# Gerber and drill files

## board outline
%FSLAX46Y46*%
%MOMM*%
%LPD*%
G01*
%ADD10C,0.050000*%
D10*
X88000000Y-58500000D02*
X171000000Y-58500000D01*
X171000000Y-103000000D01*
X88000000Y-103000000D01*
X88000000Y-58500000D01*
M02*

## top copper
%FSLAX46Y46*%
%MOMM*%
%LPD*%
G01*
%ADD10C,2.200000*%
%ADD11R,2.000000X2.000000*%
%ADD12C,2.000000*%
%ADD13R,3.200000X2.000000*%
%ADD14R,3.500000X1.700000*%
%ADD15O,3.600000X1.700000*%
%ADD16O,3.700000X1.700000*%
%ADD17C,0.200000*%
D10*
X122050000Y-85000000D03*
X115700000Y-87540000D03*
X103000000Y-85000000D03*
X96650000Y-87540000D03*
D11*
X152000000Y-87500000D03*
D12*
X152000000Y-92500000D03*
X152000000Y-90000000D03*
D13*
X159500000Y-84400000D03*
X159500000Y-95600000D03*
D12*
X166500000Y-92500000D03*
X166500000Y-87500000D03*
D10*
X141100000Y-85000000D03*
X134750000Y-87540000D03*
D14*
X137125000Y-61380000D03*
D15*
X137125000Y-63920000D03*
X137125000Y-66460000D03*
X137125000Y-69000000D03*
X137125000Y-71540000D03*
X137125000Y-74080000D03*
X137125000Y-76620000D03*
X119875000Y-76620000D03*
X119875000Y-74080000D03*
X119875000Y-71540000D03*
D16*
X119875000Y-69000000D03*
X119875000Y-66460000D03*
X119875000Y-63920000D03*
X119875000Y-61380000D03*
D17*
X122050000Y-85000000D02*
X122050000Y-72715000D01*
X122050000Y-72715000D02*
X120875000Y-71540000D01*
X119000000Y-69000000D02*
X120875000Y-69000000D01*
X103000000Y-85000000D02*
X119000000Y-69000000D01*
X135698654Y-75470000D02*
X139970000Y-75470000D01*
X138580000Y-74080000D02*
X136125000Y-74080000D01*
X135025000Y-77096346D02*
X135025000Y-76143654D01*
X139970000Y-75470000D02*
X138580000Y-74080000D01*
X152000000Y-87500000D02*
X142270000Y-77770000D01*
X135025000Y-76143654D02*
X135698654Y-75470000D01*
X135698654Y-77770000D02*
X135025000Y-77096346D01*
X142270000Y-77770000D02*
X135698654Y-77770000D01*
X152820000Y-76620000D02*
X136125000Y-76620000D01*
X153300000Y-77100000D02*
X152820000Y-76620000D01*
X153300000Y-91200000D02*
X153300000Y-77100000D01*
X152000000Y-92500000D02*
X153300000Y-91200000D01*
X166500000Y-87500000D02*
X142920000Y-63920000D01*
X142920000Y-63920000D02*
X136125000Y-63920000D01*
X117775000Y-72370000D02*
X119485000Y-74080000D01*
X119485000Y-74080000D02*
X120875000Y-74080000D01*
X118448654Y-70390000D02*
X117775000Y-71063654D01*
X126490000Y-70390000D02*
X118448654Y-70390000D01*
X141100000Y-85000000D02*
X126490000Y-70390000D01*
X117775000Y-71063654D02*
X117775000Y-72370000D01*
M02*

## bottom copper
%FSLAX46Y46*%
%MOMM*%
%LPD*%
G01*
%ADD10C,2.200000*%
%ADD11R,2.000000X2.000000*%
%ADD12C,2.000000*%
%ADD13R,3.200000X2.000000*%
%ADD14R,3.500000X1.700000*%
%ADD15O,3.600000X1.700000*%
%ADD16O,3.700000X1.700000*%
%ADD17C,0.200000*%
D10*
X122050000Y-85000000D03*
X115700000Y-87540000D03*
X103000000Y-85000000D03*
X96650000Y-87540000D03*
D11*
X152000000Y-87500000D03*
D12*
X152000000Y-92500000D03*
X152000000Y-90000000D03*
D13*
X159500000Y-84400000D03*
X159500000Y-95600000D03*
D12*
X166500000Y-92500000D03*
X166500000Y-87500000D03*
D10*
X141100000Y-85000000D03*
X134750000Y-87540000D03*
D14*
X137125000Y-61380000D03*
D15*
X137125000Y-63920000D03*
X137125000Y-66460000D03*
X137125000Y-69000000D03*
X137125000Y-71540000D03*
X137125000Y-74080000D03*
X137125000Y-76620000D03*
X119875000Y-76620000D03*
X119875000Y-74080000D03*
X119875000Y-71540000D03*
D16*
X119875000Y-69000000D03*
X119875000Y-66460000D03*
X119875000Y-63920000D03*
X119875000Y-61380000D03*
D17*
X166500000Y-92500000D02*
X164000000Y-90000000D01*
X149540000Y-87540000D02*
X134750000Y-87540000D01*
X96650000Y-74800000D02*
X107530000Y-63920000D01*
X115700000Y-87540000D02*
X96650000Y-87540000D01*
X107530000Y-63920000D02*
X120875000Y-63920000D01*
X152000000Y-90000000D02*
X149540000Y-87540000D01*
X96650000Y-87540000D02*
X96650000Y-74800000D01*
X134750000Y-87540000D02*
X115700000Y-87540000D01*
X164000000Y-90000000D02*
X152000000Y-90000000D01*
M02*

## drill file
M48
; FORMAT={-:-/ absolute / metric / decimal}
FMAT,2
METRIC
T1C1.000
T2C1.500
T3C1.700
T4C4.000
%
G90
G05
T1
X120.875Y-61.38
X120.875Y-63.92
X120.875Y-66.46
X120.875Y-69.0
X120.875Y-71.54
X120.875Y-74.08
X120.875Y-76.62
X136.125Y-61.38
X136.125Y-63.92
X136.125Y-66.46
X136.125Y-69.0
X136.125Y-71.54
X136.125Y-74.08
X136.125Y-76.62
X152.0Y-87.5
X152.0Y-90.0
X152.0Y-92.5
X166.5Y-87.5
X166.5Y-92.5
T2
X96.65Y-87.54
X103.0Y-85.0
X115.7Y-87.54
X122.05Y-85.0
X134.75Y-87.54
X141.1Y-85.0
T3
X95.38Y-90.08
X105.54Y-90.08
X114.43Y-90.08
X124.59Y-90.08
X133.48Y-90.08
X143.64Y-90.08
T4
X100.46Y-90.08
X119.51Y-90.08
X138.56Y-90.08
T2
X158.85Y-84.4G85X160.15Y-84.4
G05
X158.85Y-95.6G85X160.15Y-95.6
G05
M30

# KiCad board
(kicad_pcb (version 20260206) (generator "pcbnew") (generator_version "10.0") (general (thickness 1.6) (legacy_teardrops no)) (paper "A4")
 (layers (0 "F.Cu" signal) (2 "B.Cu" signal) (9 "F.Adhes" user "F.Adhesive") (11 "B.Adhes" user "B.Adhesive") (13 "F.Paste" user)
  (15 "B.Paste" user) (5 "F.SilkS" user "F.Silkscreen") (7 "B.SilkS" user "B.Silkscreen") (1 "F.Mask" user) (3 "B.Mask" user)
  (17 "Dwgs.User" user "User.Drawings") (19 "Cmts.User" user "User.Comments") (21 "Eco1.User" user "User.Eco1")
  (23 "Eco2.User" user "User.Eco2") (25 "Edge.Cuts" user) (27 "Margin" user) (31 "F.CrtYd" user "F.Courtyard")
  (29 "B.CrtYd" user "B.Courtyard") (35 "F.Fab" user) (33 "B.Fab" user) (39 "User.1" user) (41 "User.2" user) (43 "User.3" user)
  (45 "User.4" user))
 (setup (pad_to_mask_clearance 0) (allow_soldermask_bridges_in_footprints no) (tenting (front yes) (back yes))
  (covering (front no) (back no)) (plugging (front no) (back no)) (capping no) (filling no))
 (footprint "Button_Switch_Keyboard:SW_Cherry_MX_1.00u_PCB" (layer "F.Cu") (at 122.05 85)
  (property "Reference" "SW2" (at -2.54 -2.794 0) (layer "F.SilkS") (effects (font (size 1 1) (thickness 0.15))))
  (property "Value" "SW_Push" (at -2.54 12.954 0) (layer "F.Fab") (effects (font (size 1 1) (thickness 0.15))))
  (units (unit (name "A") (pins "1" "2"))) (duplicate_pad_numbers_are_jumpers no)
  (pad "" np_thru_hole circle (at -7.62 5.08) (size 1.7 1.7) (drill 1.7) (layers "*.Cu" "*.Mask"))
  (pad "" np_thru_hole circle (at -2.54 5.08) (size 4 4) (drill 4) (layers "*.Cu" "*.Mask"))
  (pad "" np_thru_hole circle (at 2.54 5.08) (size 1.7 1.7) (drill 1.7) (layers "*.Cu" "*.Mask"))
  (pad "1" thru_hole circle (at 0 0) (size 2.2 2.2) (drill 1.5) (layers "*.Cu" "*.Mask") (remove_unused_layers no)
   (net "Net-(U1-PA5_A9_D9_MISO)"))
  (pad "2" thru_hole circle (at -6.35 2.54) (size 2.2 2.2) (drill 1.5) (layers "*.Cu" "*.Mask") (remove_unused_layers no) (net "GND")))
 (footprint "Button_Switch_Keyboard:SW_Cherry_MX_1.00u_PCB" (layer "F.Cu") (at 103 85)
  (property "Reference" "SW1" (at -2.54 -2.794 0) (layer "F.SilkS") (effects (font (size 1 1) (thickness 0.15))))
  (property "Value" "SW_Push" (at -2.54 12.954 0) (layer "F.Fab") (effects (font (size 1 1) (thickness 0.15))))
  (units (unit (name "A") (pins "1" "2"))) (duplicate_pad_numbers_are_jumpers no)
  (pad "" np_thru_hole circle (at -7.62 5.08) (size 1.7 1.7) (drill 1.7) (layers "*.Cu" "*.Mask"))
  (pad "" np_thru_hole circle (at -2.54 5.08) (size 4 4) (drill 4) (layers "*.Cu" "*.Mask"))
  (pad "" np_thru_hole circle (at 2.54 5.08) (size 1.7 1.7) (drill 1.7) (layers "*.Cu" "*.Mask"))
  (pad "1" thru_hole circle (at 0 0) (size 2.2 2.2) (drill 1.5) (layers "*.Cu" "*.Mask") (remove_unused_layers no)
   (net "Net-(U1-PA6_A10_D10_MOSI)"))
  (pad "2" thru_hole circle (at -6.35 2.54) (size 2.2 2.2) (drill 1.5) (layers "*.Cu" "*.Mask") (remove_unused_layers no) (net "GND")))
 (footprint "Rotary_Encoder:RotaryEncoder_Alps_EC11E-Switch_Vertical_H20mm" (layer "F.Cu") (at 152 87.5)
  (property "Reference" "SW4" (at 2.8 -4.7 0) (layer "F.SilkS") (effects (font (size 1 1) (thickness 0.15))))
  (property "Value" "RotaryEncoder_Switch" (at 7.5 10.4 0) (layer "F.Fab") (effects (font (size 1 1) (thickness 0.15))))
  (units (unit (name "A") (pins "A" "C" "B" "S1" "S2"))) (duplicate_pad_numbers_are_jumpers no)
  (pad "A" thru_hole rect (at 0 0) (size 2 2) (drill 1) (layers "*.Cu" "*.Mask") (remove_unused_layers no) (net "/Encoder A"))
  (pad "B" thru_hole circle (at 0 5) (size 2 2) (drill 1) (layers "*.Cu" "*.Mask") (remove_unused_layers no) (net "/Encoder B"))
  (pad "C" thru_hole circle (at 0 2.5) (size 2 2) (drill 1) (layers "*.Cu" "*.Mask") (remove_unused_layers no) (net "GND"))
  (pad "MP" thru_hole rect (at 7.5 -3.1) (size 3.2 2) (drill oval 2.8 1.5) (layers "*.Cu" "*.Mask") (remove_unused_layers no))
  (pad "MP" thru_hole rect (at 7.5 8.1) (size 3.2 2) (drill oval 2.8 1.5) (layers "*.Cu" "*.Mask") (remove_unused_layers no))
  (pad "S1" thru_hole circle (at 14.5 5) (size 2 2) (drill 1) (layers "*.Cu" "*.Mask") (remove_unused_layers no) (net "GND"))
  (pad "S2" thru_hole circle (at 14.5 0) (size 2 2) (drill 1) (layers "*.Cu" "*.Mask") (remove_unused_layers no) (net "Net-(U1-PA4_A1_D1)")))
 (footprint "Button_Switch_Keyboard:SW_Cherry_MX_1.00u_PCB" (layer "F.Cu") (at 141.1 85)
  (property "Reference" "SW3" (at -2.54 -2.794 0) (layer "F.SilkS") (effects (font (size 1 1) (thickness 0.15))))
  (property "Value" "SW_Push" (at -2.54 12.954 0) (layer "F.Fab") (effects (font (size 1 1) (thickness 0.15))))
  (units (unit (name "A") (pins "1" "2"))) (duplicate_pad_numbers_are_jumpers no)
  (pad "" np_thru_hole circle (at -7.62 5.08) (size 1.7 1.7) (drill 1.7) (layers "*.Cu" "*.Mask"))
  (pad "" np_thru_hole circle (at -2.54 5.08) (size 4 4) (drill 4) (layers "*.Cu" "*.Mask"))
  (pad "" np_thru_hole circle (at 2.54 5.08) (size 1.7 1.7) (drill 1.7) (layers "*.Cu" "*.Mask"))
  (pad "1" thru_hole circle (at 0 0) (size 2.2 2.2) (drill 1.5) (layers "*.Cu" "*.Mask") (remove_unused_layers no)
   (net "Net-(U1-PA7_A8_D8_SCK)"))
  (pad "2" thru_hole circle (at -6.35 2.54) (size 2.2 2.2) (drill 1.5) (layers "*.Cu" "*.Mask") (remove_unused_layers no) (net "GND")))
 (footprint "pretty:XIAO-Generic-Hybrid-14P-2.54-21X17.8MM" (layer "B.Cu") (at 128.5 69 180)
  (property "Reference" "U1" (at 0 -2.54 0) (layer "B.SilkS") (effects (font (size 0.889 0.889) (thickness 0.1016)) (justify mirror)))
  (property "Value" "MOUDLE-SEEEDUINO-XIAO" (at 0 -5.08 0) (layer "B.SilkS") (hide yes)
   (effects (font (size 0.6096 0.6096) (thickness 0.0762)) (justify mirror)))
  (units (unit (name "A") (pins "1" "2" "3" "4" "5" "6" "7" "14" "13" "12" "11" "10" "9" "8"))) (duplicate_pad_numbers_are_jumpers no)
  (pad "1" thru_hole rect (at -7.625 7.62 180) (size 3.5 1.7) (drill 1 (offset -1 0)) (layers "*.Cu" "*.Mask") (remove_unused_layers no)
   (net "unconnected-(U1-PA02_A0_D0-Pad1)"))
  (pad "2" thru_hole oval (at -7.625 5.08 180) (size 3.6 1.7) (drill 1 (offset -1 0)) (layers "*.Cu" "*.Mask") (remove_unused_layers no)
   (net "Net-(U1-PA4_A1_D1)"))
  (pad "3" thru_hole oval (at -7.625 2.54 180) (size 3.6 1.7) (drill 1 (offset -1 0)) (layers "*.Cu" "*.Mask") (remove_unused_layers no)
   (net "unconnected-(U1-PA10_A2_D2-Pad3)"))
  (pad "4" thru_hole oval (at -7.625 0 180) (size 3.6 1.7) (drill 1 (offset -1 0)) (layers "*.Cu" "*.Mask") (remove_unused_layers no)
   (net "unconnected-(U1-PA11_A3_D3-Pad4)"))
  (pad "5" thru_hole oval (at -7.625 -2.54 180) (size 3.6 1.7) (drill 1 (offset -1 0)) (layers "*.Cu" "*.Mask") (remove_unused_layers no)
   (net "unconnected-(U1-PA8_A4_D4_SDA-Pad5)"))
  (pad "6" thru_hole oval (at -7.625 -5.08) (size 3.6 1.7) (drill 1 (offset 1 0)) (layers "*.Cu" "*.Mask") (remove_unused_layers no)
   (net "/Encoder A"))
  (pad "7" thru_hole oval (at -7.625 -7.62 180) (size 3.6 1.7) (drill 1 (offset -1 0)) (layers "*.Cu" "*.Mask") (remove_unused_layers no)
   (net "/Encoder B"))
  (pad "8" thru_hole oval (at 7.625 -7.62 180) (size 3.6 1.7) (drill 1 (offset 1 0)) (layers "*.Cu" "*.Mask") (remove_unused_layers no)
   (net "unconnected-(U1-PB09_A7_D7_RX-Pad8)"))
  (pad "9" thru_hole oval (at 7.625 -5.08 180) (size 3.6 1.7) (drill 1 (offset 1 0)) (layers "*.Cu" "*.Mask") (remove_unused_layers no)
   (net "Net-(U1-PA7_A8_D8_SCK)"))
  (pad "10" thru_hole oval (at 7.625 -2.54 180) (size 3.6 1.7) (drill 1 (offset 1 0)) (layers "*.Cu" "*.Mask") (remove_unused_layers no)
   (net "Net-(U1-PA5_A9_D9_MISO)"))
  (pad "11" thru_hole oval (at 7.625 0 180) (size 3.7 1.7) (drill 1 (offset 1 0)) (layers "*.Cu" "*.Mask") (remove_unused_layers no)
   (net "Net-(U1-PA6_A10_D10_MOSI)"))
  (pad "12" thru_hole oval (at 7.625 2.54 180) (size 3.7 1.7) (drill 1 (offset 1 0)) (layers "*.Cu" "*.Mask") (remove_unused_layers no)
   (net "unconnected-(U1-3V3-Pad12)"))
  (pad "13" thru_hole oval (at 7.625 5.08 180) (size 3.7 1.7) (drill 1 (offset 1 0)) (layers "*.Cu" "*.Mask") (remove_unused_layers no)
   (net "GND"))
  (pad "14" thru_hole oval (at 7.625 7.62 180) (size 3.7 1.7) (drill 1 (offset 1 0)) (layers "*.Cu" "*.Mask") (remove_unused_layers no)
   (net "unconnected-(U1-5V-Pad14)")))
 (gr_rect (start 88 58.5) (end 171 103) (stroke (width 0.05) (type default)) (fill no) (layer "Edge.Cuts"))
 (segment (start 122.05 85) (end 122.05 72.715) (width 0.2) (layer "F.Cu") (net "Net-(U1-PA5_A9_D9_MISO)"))
 (segment (start 122.05 72.715) (end 120.875 71.54) (width 0.2) (layer "F.Cu") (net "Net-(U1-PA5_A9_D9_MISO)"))
 (segment (start 166.5 92.5) (end 164 90) (width 0.2) (layer "B.Cu") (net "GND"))
 (segment (start 149.54 87.54) (end 134.75 87.54) (width 0.2) (layer "B.Cu") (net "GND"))
 (segment (start 96.65 74.8) (end 107.53 63.92) (width 0.2) (layer "B.Cu") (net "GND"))
 (segment (start 115.7 87.54) (end 96.65 87.54) (width 0.2) (layer "B.Cu") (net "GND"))
 (segment (start 107.53 63.92) (end 120.875 63.92) (width 0.2) (layer "B.Cu") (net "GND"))
 (segment (start 152 90) (end 149.54 87.54) (width 0.2) (layer "B.Cu") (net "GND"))
 (segment (start 96.65 87.54) (end 96.65 74.8) (width 0.2) (layer "B.Cu") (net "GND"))
 (segment (start 134.75 87.54) (end 115.7 87.54) (width 0.2) (layer "B.Cu") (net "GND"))
 (segment (start 164 90) (end 152 90) (width 0.2) (layer "B.Cu") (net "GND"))
 (segment (start 119 69) (end 120.875 69) (width 0.2) (layer "F.Cu") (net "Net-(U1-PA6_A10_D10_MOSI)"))
 (segment (start 103 85) (end 119 69) (width 0.2) (layer "F.Cu") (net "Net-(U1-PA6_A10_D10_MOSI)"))
 (segment (start 135.698654 75.47) (end 139.97 75.47) (width 0.2) (layer "F.Cu") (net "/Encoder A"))
 (segment (start 138.58 74.08) (end 136.125 74.08) (width 0.2) (layer "F.Cu") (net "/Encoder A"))
 (segment (start 135.025 77.096346) (end 135.025 76.143654) (width 0.2) (layer "F.Cu") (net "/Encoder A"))
 (segment (start 139.97 75.47) (end 138.58 74.08) (width 0.2) (layer "F.Cu") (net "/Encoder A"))
 (segment (start 152 87.5) (end 142.27 77.77) (width 0.2) (layer "F.Cu") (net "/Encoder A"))
 (segment (start 135.025 76.143654) (end 135.698654 75.47) (width 0.2) (layer "F.Cu") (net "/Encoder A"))
 (segment (start 135.698654 77.77) (end 135.025 77.096346) (width 0.2) (layer "F.Cu") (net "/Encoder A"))
 (segment (start 142.27 77.77) (end 135.698654 77.77) (width 0.2) (layer "F.Cu") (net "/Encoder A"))
 (segment (start 152.82 76.62) (end 136.125 76.62) (width 0.2) (layer "F.Cu") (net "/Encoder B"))
 (segment (start 153.3 77.1) (end 152.82 76.62) (width 0.2) (layer "F.Cu") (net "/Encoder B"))
 (segment (start 153.3 91.2) (end 153.3 77.1) (width 0.2) (layer "F.Cu") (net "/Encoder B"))
 (segment (start 152 92.5) (end 153.3 91.2) (width 0.2) (layer "F.Cu") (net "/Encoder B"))
 (segment (start 166.5 87.5) (end 142.92 63.92) (width 0.2) (layer "F.Cu") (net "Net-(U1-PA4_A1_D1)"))
 (segment (start 142.92 63.92) (end 136.125 63.92) (width 0.2) (layer "F.Cu") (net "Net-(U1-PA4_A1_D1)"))
 (segment (start 117.775 72.37) (end 119.485 74.08) (width 0.2) (layer "F.Cu") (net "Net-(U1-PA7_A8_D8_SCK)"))
 (segment (start 119.485 74.08) (end 120.875 74.08) (width 0.2) (layer "F.Cu") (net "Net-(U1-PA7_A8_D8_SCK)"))
 (segment (start 118.448654 70.39) (end 117.775 71.063654) (width 0.2) (layer "F.Cu") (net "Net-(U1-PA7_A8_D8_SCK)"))
 (segment (start 126.49 70.39) (end 118.448654 70.39) (width 0.2) (layer "F.Cu") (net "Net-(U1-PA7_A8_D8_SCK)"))
 (segment (start 141.1 85) (end 126.49 70.39) (width 0.2) (layer "F.Cu") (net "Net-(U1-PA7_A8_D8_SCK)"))
 (segment (start 117.775 71.063654) (end 117.775 72.37) (width 0.2) (layer "F.Cu") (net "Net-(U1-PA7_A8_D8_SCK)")))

